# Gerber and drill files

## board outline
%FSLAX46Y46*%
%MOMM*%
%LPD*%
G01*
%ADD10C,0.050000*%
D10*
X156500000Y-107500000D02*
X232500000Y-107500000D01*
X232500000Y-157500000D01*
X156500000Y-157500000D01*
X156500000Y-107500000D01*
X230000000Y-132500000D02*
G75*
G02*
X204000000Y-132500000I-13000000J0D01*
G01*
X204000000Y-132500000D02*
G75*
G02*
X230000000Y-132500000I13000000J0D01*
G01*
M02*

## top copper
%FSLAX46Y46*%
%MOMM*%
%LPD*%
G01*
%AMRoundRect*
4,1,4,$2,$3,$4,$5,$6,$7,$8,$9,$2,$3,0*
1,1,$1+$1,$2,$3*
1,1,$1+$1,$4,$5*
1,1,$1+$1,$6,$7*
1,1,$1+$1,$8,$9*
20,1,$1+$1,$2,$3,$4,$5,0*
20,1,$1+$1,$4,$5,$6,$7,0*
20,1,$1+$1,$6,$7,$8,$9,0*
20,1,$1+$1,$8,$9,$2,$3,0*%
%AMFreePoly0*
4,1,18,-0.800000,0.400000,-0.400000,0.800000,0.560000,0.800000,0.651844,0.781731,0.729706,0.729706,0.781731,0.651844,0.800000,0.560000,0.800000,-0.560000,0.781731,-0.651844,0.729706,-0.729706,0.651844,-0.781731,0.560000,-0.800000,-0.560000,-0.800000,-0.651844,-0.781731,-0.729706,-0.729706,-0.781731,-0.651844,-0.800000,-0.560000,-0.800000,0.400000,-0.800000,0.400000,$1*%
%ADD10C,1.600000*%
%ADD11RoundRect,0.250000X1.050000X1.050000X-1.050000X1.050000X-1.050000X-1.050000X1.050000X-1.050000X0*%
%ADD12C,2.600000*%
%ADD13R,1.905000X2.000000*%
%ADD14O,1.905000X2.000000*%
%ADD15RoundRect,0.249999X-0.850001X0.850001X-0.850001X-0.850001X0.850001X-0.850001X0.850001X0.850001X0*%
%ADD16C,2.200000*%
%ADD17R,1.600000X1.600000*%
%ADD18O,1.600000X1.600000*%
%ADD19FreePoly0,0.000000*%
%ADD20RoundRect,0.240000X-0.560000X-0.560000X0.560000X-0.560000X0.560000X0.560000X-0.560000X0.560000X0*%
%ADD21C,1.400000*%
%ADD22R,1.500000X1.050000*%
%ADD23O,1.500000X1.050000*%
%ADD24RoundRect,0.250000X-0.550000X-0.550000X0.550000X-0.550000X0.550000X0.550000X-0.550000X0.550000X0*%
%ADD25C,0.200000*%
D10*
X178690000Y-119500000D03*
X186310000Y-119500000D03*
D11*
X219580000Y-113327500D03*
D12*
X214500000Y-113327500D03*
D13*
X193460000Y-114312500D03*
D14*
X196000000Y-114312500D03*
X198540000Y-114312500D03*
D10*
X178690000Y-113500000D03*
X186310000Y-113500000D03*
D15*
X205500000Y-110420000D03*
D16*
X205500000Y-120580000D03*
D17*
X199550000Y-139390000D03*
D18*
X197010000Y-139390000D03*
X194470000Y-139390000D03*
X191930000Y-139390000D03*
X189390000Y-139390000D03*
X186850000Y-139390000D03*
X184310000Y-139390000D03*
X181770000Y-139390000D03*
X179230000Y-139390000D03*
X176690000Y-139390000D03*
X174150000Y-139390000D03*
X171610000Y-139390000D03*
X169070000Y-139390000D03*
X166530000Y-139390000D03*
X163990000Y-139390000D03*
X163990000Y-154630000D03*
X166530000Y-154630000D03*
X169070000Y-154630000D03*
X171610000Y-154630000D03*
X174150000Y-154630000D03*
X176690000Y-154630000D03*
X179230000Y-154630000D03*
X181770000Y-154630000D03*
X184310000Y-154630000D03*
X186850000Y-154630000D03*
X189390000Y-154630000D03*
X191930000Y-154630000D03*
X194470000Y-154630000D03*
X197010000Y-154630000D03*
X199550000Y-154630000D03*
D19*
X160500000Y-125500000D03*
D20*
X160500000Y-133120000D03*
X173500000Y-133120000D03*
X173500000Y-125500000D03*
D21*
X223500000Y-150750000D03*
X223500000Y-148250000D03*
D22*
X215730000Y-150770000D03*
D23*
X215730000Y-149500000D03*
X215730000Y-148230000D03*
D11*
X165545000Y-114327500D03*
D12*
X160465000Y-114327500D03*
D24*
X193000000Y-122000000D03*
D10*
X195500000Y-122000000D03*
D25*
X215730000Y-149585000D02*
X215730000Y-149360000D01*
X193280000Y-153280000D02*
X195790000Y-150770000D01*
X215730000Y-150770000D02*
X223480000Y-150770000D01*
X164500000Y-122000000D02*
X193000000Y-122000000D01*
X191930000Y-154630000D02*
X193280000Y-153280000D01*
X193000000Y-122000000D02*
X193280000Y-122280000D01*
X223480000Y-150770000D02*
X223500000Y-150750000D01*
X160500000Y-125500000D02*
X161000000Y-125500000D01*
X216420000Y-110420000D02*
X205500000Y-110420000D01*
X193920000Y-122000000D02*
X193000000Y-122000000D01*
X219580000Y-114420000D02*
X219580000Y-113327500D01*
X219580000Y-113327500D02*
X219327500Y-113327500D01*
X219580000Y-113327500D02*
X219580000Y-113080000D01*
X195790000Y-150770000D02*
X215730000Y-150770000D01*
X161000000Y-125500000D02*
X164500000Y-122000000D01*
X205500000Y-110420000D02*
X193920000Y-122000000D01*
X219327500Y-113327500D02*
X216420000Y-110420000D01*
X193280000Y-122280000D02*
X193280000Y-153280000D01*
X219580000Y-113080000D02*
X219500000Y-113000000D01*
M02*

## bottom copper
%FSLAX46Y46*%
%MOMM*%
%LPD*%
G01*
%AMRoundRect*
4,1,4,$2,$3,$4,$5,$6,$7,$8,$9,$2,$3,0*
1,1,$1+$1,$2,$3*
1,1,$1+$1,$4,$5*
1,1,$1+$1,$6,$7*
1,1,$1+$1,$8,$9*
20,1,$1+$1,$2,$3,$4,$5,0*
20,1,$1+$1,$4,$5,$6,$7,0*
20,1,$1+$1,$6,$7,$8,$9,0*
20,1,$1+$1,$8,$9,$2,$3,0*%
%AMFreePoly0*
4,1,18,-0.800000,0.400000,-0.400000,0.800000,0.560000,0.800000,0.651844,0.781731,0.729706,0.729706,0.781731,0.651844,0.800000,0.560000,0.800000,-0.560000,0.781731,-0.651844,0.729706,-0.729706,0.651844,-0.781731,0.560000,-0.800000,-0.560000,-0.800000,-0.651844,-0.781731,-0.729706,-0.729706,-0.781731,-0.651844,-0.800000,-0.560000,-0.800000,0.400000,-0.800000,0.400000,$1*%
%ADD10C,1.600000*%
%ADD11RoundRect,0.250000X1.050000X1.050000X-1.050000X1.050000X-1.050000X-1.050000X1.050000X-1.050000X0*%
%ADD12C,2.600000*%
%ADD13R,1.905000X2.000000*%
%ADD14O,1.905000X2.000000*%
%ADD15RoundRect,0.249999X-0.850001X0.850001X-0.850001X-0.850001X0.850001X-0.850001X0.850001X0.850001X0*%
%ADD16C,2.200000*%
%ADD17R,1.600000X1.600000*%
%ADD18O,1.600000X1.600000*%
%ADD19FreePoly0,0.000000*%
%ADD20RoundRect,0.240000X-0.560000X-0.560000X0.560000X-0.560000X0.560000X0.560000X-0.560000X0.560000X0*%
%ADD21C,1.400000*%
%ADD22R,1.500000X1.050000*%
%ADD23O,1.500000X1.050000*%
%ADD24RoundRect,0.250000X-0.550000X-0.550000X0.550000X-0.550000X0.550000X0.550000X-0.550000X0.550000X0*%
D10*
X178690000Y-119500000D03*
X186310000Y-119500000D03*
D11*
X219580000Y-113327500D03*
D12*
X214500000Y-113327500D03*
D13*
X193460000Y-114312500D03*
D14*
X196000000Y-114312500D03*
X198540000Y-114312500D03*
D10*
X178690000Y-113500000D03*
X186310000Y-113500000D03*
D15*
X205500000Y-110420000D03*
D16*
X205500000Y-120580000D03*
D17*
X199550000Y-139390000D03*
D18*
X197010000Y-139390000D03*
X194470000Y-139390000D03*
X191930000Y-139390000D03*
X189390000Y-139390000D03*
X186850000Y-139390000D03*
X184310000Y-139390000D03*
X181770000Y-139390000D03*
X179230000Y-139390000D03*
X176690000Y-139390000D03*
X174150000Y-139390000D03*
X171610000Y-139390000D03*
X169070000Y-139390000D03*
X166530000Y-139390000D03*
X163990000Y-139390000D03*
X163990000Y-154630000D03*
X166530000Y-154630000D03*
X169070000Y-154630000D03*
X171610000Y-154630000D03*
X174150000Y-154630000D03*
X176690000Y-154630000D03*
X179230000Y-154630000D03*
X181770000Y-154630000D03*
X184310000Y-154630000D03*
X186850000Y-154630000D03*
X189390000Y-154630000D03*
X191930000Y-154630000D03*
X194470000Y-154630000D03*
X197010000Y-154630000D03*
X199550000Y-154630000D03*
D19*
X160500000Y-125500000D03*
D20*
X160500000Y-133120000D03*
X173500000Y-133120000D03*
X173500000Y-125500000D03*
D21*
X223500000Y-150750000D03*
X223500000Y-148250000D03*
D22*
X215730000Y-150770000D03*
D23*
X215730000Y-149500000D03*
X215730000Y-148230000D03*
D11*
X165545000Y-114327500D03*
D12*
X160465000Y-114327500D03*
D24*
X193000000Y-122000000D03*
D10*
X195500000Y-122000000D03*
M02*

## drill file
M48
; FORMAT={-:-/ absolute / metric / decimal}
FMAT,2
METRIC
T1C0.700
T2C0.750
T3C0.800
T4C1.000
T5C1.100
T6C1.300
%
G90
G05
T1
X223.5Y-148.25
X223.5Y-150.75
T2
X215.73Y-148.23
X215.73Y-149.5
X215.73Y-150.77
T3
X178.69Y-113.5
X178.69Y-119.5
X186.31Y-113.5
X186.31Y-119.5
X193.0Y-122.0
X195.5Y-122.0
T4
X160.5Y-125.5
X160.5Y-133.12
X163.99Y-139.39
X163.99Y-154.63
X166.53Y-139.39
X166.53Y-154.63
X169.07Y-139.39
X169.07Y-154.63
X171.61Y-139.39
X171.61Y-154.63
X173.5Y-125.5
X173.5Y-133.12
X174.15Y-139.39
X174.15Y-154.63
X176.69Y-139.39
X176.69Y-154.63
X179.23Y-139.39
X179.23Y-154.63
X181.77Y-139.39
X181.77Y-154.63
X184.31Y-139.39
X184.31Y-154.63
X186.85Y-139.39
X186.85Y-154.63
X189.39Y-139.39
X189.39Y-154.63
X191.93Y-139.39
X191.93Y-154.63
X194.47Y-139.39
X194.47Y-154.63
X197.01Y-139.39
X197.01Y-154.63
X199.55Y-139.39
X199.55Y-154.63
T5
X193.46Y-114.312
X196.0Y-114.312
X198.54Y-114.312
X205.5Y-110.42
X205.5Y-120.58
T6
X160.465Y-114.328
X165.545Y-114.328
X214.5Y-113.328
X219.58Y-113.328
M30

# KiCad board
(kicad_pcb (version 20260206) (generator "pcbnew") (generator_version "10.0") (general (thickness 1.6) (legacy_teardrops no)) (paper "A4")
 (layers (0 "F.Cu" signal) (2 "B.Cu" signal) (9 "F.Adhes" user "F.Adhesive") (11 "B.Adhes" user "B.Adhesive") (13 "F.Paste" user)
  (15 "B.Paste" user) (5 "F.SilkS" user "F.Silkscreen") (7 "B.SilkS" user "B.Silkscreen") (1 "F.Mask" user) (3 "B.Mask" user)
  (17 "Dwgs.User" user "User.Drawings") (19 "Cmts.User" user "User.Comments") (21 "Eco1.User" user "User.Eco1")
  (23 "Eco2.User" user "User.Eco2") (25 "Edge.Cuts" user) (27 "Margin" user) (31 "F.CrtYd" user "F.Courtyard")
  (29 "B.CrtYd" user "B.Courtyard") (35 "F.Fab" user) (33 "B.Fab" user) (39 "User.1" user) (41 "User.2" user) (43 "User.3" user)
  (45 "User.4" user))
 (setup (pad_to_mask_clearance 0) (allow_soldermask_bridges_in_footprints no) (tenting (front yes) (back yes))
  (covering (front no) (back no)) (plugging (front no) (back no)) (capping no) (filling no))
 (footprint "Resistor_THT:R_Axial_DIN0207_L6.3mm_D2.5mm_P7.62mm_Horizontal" (layer "F.Cu") (at 178.69 119.5)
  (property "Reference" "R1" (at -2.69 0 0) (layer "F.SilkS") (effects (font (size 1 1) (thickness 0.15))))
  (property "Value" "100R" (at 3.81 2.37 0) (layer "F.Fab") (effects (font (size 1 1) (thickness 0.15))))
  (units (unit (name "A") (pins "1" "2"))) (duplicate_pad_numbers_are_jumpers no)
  (pad "1" thru_hole circle (at 0 0) (size 1.6 1.6) (drill 0.8) (layers "*.Cu" "*.Mask") (remove_unused_layers no) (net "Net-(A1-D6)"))
  (pad "2" thru_hole circle (at 7.62 0) (size 1.6 1.6) (drill 0.8) (layers "*.Cu" "*.Mask") (remove_unused_layers no) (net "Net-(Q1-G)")))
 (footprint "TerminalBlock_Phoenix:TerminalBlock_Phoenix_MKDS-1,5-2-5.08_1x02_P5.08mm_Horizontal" (layer "F.Cu") (at 219.58 113.3275 180)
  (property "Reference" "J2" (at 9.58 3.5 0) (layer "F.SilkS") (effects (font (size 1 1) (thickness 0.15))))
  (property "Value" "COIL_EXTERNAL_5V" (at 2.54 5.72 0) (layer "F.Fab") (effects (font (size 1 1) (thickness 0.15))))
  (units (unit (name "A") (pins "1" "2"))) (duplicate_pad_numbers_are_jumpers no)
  (pad "1" thru_hole roundrect (at 0 0 180) (size 2.6 2.6) (drill 1.3) (layers "*.Cu" "*.Mask") (remove_unused_layers no)
   (roundrect_rratio 0.096154) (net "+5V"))
  (pad "2" thru_hole circle (at 5.08 0 180) (size 2.6 2.6) (drill 1.3) (layers "*.Cu" "*.Mask") (remove_unused_layers no) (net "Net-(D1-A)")))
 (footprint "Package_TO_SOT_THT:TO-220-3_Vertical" (layer "F.Cu") (at 193.46 114.3125)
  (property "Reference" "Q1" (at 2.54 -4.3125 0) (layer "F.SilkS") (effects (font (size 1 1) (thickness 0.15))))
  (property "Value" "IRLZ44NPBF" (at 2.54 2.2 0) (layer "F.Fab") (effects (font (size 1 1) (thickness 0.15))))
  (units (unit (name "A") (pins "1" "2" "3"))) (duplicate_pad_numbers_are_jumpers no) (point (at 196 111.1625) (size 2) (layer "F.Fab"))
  (pad "1" thru_hole rect (at 0 0) (size 1.905 2) (drill 1.1) (layers "*.Cu" "*.Mask") (remove_unused_layers no) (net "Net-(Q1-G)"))
  (pad "2" thru_hole oval (at 2.54 0) (size 1.905 2) (drill 1.1) (layers "*.Cu" "*.Mask") (remove_unused_layers no) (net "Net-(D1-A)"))
  (pad "3" thru_hole oval (at 5.08 0) (size 1.905 2) (drill 1.1) (layers "*.Cu" "*.Mask") (remove_unused_layers no) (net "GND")))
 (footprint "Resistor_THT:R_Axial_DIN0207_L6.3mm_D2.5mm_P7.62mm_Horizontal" (layer "F.Cu") (at 178.69 113.5)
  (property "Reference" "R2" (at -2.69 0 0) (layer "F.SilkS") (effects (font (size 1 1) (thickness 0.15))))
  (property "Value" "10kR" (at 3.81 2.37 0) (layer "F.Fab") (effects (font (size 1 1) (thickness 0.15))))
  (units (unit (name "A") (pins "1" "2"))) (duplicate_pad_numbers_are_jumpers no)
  (pad "1" thru_hole circle (at 0 0) (size 1.6 1.6) (drill 0.8) (layers "*.Cu" "*.Mask") (remove_unused_layers no) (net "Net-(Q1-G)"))
  (pad "2" thru_hole circle (at 7.62 0) (size 1.6 1.6) (drill 0.8) (layers "*.Cu" "*.Mask") (remove_unused_layers no) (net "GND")))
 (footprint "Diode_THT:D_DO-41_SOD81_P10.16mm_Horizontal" (layer "F.Cu") (at 205.5 110.42 -90)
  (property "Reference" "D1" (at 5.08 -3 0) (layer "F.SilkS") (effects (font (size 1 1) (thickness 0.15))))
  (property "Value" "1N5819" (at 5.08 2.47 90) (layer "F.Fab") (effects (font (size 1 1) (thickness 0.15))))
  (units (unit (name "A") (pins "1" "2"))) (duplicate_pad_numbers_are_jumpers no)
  (pad "1" thru_hole roundrect (at 0 0 270) (size 2.2 2.2) (drill 1.1) (layers "*.Cu" "*.Mask") (remove_unused_layers no)
   (roundrect_rratio 0.113636) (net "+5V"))
  (pad "2" thru_hole circle (at 10.16 0 270) (size 2.2 2.2) (drill 1.1) (layers "*.Cu" "*.Mask") (remove_unused_layers no)
   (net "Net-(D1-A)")))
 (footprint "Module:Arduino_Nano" (layer "F.Cu") (at 199.55 139.39 -90)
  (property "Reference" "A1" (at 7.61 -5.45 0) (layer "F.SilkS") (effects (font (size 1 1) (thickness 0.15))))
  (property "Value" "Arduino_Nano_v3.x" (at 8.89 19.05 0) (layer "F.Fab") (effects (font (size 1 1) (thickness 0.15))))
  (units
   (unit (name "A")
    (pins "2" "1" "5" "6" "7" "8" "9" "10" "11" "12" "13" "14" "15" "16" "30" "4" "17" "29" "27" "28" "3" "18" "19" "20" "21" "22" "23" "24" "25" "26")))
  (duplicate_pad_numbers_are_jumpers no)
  (pad "1" thru_hole rect (at 0 0 270) (size 1.6 1.6) (drill 1) (layers "*.Cu" "*.Mask") (remove_unused_layers no)
   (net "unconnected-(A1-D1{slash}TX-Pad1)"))
  (pad "2" thru_hole oval (at 0 2.54 270) (size 1.6 1.6) (drill 1) (layers "*.Cu" "*.Mask") (remove_unused_layers no)
   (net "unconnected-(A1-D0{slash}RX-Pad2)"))
  (pad "3" thru_hole oval (at 0 5.08 270) (size 1.6 1.6) (drill 1) (layers "*.Cu" "*.Mask") (remove_unused_layers no)
   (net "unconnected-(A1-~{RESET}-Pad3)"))
  (pad "4" thru_hole oval (at 0 7.62 270) (size 1.6 1.6) (drill 1) (layers "*.Cu" "*.Mask") (remove_unused_layers no) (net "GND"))
  (pad "5" thru_hole oval (at 0 10.16 270) (size 1.6 1.6) (drill 1) (layers "*.Cu" "*.Mask") (remove_unused_layers no)
   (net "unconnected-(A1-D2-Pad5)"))
  (pad "6" thru_hole oval (at 0 12.7 270) (size 1.6 1.6) (drill 1) (layers "*.Cu" "*.Mask") (remove_unused_layers no)
   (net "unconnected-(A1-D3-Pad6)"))
  (pad "7" thru_hole oval (at 0 15.24 270) (size 1.6 1.6) (drill 1) (layers "*.Cu" "*.Mask") (remove_unused_layers no)
   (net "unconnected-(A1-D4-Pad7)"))
  (pad "8" thru_hole oval (at 0 17.78 270) (size 1.6 1.6) (drill 1) (layers "*.Cu" "*.Mask") (remove_unused_layers no)
   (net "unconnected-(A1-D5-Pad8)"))
  (pad "9" thru_hole oval (at 0 20.32 270) (size 1.6 1.6) (drill 1) (layers "*.Cu" "*.Mask") (remove_unused_layers no) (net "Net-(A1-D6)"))
  (pad "10" thru_hole oval (at 0 22.86 270) (size 1.6 1.6) (drill 1) (layers "*.Cu" "*.Mask") (remove_unused_layers no)
   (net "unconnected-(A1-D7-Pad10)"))
  (pad "11" thru_hole oval (at 0 25.4 270) (size 1.6 1.6) (drill 1) (layers "*.Cu" "*.Mask") (remove_unused_layers no)
   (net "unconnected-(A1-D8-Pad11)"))
  (pad "12" thru_hole oval (at 0 27.94 270) (size 1.6 1.6) (drill 1) (layers "*.Cu" "*.Mask") (remove_unused_layers no)
   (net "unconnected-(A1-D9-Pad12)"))
  (pad "13" thru_hole oval (at 0 30.48 270) (size 1.6 1.6) (drill 1) (layers "*.Cu" "*.Mask") (remove_unused_layers no)
   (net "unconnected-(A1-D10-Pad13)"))
  (pad "14" thru_hole oval (at 0 33.02 270) (size 1.6 1.6) (drill 1) (layers "*.Cu" "*.Mask") (remove_unused_layers no)
   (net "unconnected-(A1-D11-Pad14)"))
  (pad "15" thru_hole oval (at 0 35.56 270) (size 1.6 1.6) (drill 1) (layers "*.Cu" "*.Mask") (remove_unused_layers no)
   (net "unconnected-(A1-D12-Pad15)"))
  (pad "16" thru_hole oval (at 15.24 35.56 270) (size 1.6 1.6) (drill 1) (layers "*.Cu" "*.Mask") (remove_unused_layers no)
   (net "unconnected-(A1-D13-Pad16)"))
  (pad "17" thru_hole oval (at 15.24 33.02 270) (size 1.6 1.6) (drill 1) (layers "*.Cu" "*.Mask") (remove_unused_layers no)
   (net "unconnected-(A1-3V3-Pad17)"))
  (pad "18" thru_hole oval (at 15.24 30.48 270) (size 1.6 1.6) (drill 1) (layers "*.Cu" "*.Mask") (remove_unused_layers no)
   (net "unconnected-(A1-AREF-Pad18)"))
  (pad "19" thru_hole oval (at 15.24 27.94 270) (size 1.6 1.6) (drill 1) (layers "*.Cu" "*.Mask") (remove_unused_layers no)
   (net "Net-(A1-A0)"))
  (pad "20" thru_hole oval (at 15.24 25.4 270) (size 1.6 1.6) (drill 1) (layers "*.Cu" "*.Mask") (remove_unused_layers no)
   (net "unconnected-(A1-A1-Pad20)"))
  (pad "21" thru_hole oval (at 15.24 22.86 270) (size 1.6 1.6) (drill 1) (layers "*.Cu" "*.Mask") (remove_unused_layers no)
   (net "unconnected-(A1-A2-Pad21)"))
  (pad "22" thru_hole oval (at 15.24 20.32 270) (size 1.6 1.6) (drill 1) (layers "*.Cu" "*.Mask") (remove_unused_layers no)
   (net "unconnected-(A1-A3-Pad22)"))
  (pad "23" thru_hole oval (at 15.24 17.78 270) (size 1.6 1.6) (drill 1) (layers "*.Cu" "*.Mask") (remove_unused_layers no)
   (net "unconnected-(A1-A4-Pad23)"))
  (pad "24" thru_hole oval (at 15.24 15.24 270) (size 1.6 1.6) (drill 1) (layers "*.Cu" "*.Mask") (remove_unused_layers no)
   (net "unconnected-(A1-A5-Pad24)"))
  (pad "25" thru_hole oval (at 15.24 12.7 270) (size 1.6 1.6) (drill 1) (layers "*.Cu" "*.Mask") (remove_unused_layers no)
   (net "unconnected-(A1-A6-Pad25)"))
  (pad "26" thru_hole oval (at 15.24 10.16 270) (size 1.6 1.6) (drill 1) (layers "*.Cu" "*.Mask") (remove_unused_layers no)
   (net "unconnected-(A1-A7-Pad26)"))
  (pad "27" thru_hole oval (at 15.24 7.62 270) (size 1.6 1.6) (drill 1) (layers "*.Cu" "*.Mask") (remove_unused_layers no) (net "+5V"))
  (pad "28" thru_hole oval (at 15.24 5.08 270) (size 1.6 1.6) (drill 1) (layers "*.Cu" "*.Mask") (remove_unused_layers no)
   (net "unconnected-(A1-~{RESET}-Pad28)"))
  (pad "29" thru_hole oval (at 15.24 2.54 270) (size 1.6 1.6) (drill 1) (layers "*.Cu" "*.Mask") (remove_unused_layers no) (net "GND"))
  (pad "30" thru_hole oval (at 15.24 0 270) (size 1.6 1.6) (drill 1) (layers "*.Cu" "*.Mask") (remove_unused_layers no)
   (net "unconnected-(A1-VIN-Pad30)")))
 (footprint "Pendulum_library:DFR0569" (layer "F.Cu") (at 167 129.31)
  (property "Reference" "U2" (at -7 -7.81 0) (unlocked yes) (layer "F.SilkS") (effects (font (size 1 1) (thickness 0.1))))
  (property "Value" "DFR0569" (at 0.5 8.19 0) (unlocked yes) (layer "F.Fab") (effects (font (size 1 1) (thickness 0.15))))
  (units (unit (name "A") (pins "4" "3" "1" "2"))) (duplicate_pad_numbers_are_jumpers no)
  (pad "1" thru_hole roundrect (at -6.5 -3.81) (size 1.6 1.6) (drill 1) (layers "*.Cu" "*.Mask") (remove_unused_layers no)
   (roundrect_rratio 0.15) (chamfer_ratio 0.25) (chamfer top_left) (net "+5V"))
  (pad "2" thru_hole roundrect (at -6.5 3.81) (size 1.6 1.6) (drill 1) (layers "*.Cu" "*.Mask") (remove_unused_layers no)
   (roundrect_rratio 0.15) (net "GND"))
  (pad "3" thru_hole roundrect (at 6.5 3.81) (size 1.6 1.6) (drill 1) (layers "*.Cu" "*.Mask") (remove_unused_layers no)
   (roundrect_rratio 0.15) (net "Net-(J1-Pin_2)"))
  (pad "4" thru_hole roundrect (at 6.5 -3.81) (size 1.6 1.6) (drill 1) (layers "*.Cu" "*.Mask") (remove_unused_layers no)
   (roundrect_rratio 0.15) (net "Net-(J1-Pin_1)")))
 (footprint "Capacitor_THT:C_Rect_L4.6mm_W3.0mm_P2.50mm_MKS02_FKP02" (layer "F.Cu") (at 223.5 150.75 90)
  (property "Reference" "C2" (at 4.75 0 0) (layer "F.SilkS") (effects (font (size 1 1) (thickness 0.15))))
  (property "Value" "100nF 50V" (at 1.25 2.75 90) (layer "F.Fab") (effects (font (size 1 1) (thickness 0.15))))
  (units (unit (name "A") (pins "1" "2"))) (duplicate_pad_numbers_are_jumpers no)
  (pad "1" thru_hole circle (at 0 0 90) (size 1.4 1.4) (drill 0.7) (layers "*.Cu" "*.Mask") (remove_unused_layers no) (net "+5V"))
  (pad "2" thru_hole circle (at 2.5 0 90) (size 1.4 1.4) (drill 0.7) (layers "*.Cu" "*.Mask") (remove_unused_layers no) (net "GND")))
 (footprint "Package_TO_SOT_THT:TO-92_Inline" (layer "F.Cu") (at 215.73 150.77 90)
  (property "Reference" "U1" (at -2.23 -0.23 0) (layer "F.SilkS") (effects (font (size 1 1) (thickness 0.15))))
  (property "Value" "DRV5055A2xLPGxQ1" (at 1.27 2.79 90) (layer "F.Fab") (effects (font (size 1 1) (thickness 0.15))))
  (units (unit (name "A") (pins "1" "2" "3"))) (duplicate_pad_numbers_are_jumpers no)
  (pad "1" thru_hole rect (at 0 0 90) (size 1.05 1.5) (drill 0.75) (layers "*.Cu" "*.Mask") (remove_unused_layers no) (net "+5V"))
  (pad "2" thru_hole oval (at 1.27 0 90) (size 1.05 1.5) (drill 0.75) (layers "*.Cu" "*.Mask") (remove_unused_layers no) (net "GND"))
  (pad "3" thru_hole oval (at 2.54 0 90) (size 1.05 1.5) (drill 0.75) (layers "*.Cu" "*.Mask") (remove_unused_layers no) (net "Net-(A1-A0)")))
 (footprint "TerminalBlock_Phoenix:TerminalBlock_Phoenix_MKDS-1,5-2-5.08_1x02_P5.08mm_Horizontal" (layer "F.Cu") (at 165.545 114.3275 180)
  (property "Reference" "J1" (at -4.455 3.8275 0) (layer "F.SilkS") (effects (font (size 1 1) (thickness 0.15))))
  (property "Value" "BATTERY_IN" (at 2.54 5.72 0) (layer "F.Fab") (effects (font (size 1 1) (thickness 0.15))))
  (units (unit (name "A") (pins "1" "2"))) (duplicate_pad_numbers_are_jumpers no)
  (pad "1" thru_hole roundrect (at 0 0 180) (size 2.6 2.6) (drill 1.3) (layers "*.Cu" "*.Mask") (remove_unused_layers no)
   (roundrect_rratio 0.096154) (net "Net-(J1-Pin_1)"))
  (pad "2" thru_hole circle (at 5.08 0 180) (size 2.6 2.6) (drill 1.3) (layers "*.Cu" "*.Mask") (remove_unused_layers no)
   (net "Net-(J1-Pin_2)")))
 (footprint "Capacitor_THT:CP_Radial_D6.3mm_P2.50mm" (layer "F.Cu") (at 193 122)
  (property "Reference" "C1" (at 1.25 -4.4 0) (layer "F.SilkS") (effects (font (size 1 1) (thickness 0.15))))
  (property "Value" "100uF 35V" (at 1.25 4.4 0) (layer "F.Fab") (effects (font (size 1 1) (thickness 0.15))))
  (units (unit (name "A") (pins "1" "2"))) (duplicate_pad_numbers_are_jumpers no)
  (pad "1" thru_hole roundrect (at 0 0) (size 1.6 1.6) (drill 0.8) (layers "*.Cu" "*.Mask") (remove_unused_layers no)
   (roundrect_rratio 0.15625) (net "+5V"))
  (pad "2" thru_hole circle (at 2.5 0) (size 1.6 1.6) (drill 0.8) (layers "*.Cu" "*.Mask") (remove_unused_layers no) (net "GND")))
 (gr_rect (start 156.5 107.5) (end 232.5 157.5) (stroke (width 0.05) (type solid)) (fill no) (layer "Edge.Cuts"))
 (gr_circle (center 217 132.5) (end 230 132.5) (stroke (width 0.05) (type default)) (fill no) (layer "Edge.Cuts"))
 (segment (start 215.73 149.585) (end 215.73 149.36) (width 0.2) (layer "F.Cu") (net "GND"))
 (segment (start 193.28 153.28) (end 195.79 150.77) (width 0.2) (layer "F.Cu") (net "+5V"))
 (segment (start 215.73 150.77) (end 223.48 150.77) (width 0.2) (layer "F.Cu") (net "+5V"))
 (segment (start 164.5 122) (end 193 122) (width 0.2) (layer "F.Cu") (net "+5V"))
 (segment (start 191.93 154.63) (end 193.28 153.28) (width 0.2) (layer "F.Cu") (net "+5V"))
 (segment (start 193 122) (end 193.28 122.28) (width 0.2) (layer "F.Cu") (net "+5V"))
 (segment (start 223.48 150.77) (end 223.5 150.75) (width 0.2) (layer "F.Cu") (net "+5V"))
 (segment (start 160.5 125.5) (end 161 125.5) (width 0.2) (layer "F.Cu") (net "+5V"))
 (segment (start 216.42 110.42) (end 205.5 110.42) (width 0.2) (layer "F.Cu") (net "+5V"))
 (segment (start 193.92 122) (end 193 122) (width 0.2) (layer "F.Cu") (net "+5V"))
 (segment (start 219.58 114.42) (end 219.58 113.3275) (width 0.2) (layer "F.Cu") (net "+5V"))
 (segment (start 219.58 113.3275) (end 219.3275 113.3275) (width 0.2) (layer "F.Cu") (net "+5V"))
 (segment (start 219.58 113.3275) (end 219.58 113.08) (width 0.2) (layer "F.Cu") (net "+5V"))
 (segment (start 195.79 150.77) (end 215.73 150.77) (width 0.2) (layer "F.Cu") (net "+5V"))
 (segment (start 161 125.5) (end 164.5 122) (width 0.2) (layer "F.Cu") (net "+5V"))
 (segment (start 205.5 110.42) (end 193.92 122) (width 0.2) (layer "F.Cu") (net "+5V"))
 (segment (start 219.3275 113.3275) (end 216.42 110.42) (width 0.2) (layer "F.Cu") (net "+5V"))
 (segment (start 193.28 122.28) (end 193.28 153.28) (width 0.2) (layer "F.Cu") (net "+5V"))
 (segment (start 219.58 113.08) (end 219.5 113) (width 0.2) (layer "F.Cu") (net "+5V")))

